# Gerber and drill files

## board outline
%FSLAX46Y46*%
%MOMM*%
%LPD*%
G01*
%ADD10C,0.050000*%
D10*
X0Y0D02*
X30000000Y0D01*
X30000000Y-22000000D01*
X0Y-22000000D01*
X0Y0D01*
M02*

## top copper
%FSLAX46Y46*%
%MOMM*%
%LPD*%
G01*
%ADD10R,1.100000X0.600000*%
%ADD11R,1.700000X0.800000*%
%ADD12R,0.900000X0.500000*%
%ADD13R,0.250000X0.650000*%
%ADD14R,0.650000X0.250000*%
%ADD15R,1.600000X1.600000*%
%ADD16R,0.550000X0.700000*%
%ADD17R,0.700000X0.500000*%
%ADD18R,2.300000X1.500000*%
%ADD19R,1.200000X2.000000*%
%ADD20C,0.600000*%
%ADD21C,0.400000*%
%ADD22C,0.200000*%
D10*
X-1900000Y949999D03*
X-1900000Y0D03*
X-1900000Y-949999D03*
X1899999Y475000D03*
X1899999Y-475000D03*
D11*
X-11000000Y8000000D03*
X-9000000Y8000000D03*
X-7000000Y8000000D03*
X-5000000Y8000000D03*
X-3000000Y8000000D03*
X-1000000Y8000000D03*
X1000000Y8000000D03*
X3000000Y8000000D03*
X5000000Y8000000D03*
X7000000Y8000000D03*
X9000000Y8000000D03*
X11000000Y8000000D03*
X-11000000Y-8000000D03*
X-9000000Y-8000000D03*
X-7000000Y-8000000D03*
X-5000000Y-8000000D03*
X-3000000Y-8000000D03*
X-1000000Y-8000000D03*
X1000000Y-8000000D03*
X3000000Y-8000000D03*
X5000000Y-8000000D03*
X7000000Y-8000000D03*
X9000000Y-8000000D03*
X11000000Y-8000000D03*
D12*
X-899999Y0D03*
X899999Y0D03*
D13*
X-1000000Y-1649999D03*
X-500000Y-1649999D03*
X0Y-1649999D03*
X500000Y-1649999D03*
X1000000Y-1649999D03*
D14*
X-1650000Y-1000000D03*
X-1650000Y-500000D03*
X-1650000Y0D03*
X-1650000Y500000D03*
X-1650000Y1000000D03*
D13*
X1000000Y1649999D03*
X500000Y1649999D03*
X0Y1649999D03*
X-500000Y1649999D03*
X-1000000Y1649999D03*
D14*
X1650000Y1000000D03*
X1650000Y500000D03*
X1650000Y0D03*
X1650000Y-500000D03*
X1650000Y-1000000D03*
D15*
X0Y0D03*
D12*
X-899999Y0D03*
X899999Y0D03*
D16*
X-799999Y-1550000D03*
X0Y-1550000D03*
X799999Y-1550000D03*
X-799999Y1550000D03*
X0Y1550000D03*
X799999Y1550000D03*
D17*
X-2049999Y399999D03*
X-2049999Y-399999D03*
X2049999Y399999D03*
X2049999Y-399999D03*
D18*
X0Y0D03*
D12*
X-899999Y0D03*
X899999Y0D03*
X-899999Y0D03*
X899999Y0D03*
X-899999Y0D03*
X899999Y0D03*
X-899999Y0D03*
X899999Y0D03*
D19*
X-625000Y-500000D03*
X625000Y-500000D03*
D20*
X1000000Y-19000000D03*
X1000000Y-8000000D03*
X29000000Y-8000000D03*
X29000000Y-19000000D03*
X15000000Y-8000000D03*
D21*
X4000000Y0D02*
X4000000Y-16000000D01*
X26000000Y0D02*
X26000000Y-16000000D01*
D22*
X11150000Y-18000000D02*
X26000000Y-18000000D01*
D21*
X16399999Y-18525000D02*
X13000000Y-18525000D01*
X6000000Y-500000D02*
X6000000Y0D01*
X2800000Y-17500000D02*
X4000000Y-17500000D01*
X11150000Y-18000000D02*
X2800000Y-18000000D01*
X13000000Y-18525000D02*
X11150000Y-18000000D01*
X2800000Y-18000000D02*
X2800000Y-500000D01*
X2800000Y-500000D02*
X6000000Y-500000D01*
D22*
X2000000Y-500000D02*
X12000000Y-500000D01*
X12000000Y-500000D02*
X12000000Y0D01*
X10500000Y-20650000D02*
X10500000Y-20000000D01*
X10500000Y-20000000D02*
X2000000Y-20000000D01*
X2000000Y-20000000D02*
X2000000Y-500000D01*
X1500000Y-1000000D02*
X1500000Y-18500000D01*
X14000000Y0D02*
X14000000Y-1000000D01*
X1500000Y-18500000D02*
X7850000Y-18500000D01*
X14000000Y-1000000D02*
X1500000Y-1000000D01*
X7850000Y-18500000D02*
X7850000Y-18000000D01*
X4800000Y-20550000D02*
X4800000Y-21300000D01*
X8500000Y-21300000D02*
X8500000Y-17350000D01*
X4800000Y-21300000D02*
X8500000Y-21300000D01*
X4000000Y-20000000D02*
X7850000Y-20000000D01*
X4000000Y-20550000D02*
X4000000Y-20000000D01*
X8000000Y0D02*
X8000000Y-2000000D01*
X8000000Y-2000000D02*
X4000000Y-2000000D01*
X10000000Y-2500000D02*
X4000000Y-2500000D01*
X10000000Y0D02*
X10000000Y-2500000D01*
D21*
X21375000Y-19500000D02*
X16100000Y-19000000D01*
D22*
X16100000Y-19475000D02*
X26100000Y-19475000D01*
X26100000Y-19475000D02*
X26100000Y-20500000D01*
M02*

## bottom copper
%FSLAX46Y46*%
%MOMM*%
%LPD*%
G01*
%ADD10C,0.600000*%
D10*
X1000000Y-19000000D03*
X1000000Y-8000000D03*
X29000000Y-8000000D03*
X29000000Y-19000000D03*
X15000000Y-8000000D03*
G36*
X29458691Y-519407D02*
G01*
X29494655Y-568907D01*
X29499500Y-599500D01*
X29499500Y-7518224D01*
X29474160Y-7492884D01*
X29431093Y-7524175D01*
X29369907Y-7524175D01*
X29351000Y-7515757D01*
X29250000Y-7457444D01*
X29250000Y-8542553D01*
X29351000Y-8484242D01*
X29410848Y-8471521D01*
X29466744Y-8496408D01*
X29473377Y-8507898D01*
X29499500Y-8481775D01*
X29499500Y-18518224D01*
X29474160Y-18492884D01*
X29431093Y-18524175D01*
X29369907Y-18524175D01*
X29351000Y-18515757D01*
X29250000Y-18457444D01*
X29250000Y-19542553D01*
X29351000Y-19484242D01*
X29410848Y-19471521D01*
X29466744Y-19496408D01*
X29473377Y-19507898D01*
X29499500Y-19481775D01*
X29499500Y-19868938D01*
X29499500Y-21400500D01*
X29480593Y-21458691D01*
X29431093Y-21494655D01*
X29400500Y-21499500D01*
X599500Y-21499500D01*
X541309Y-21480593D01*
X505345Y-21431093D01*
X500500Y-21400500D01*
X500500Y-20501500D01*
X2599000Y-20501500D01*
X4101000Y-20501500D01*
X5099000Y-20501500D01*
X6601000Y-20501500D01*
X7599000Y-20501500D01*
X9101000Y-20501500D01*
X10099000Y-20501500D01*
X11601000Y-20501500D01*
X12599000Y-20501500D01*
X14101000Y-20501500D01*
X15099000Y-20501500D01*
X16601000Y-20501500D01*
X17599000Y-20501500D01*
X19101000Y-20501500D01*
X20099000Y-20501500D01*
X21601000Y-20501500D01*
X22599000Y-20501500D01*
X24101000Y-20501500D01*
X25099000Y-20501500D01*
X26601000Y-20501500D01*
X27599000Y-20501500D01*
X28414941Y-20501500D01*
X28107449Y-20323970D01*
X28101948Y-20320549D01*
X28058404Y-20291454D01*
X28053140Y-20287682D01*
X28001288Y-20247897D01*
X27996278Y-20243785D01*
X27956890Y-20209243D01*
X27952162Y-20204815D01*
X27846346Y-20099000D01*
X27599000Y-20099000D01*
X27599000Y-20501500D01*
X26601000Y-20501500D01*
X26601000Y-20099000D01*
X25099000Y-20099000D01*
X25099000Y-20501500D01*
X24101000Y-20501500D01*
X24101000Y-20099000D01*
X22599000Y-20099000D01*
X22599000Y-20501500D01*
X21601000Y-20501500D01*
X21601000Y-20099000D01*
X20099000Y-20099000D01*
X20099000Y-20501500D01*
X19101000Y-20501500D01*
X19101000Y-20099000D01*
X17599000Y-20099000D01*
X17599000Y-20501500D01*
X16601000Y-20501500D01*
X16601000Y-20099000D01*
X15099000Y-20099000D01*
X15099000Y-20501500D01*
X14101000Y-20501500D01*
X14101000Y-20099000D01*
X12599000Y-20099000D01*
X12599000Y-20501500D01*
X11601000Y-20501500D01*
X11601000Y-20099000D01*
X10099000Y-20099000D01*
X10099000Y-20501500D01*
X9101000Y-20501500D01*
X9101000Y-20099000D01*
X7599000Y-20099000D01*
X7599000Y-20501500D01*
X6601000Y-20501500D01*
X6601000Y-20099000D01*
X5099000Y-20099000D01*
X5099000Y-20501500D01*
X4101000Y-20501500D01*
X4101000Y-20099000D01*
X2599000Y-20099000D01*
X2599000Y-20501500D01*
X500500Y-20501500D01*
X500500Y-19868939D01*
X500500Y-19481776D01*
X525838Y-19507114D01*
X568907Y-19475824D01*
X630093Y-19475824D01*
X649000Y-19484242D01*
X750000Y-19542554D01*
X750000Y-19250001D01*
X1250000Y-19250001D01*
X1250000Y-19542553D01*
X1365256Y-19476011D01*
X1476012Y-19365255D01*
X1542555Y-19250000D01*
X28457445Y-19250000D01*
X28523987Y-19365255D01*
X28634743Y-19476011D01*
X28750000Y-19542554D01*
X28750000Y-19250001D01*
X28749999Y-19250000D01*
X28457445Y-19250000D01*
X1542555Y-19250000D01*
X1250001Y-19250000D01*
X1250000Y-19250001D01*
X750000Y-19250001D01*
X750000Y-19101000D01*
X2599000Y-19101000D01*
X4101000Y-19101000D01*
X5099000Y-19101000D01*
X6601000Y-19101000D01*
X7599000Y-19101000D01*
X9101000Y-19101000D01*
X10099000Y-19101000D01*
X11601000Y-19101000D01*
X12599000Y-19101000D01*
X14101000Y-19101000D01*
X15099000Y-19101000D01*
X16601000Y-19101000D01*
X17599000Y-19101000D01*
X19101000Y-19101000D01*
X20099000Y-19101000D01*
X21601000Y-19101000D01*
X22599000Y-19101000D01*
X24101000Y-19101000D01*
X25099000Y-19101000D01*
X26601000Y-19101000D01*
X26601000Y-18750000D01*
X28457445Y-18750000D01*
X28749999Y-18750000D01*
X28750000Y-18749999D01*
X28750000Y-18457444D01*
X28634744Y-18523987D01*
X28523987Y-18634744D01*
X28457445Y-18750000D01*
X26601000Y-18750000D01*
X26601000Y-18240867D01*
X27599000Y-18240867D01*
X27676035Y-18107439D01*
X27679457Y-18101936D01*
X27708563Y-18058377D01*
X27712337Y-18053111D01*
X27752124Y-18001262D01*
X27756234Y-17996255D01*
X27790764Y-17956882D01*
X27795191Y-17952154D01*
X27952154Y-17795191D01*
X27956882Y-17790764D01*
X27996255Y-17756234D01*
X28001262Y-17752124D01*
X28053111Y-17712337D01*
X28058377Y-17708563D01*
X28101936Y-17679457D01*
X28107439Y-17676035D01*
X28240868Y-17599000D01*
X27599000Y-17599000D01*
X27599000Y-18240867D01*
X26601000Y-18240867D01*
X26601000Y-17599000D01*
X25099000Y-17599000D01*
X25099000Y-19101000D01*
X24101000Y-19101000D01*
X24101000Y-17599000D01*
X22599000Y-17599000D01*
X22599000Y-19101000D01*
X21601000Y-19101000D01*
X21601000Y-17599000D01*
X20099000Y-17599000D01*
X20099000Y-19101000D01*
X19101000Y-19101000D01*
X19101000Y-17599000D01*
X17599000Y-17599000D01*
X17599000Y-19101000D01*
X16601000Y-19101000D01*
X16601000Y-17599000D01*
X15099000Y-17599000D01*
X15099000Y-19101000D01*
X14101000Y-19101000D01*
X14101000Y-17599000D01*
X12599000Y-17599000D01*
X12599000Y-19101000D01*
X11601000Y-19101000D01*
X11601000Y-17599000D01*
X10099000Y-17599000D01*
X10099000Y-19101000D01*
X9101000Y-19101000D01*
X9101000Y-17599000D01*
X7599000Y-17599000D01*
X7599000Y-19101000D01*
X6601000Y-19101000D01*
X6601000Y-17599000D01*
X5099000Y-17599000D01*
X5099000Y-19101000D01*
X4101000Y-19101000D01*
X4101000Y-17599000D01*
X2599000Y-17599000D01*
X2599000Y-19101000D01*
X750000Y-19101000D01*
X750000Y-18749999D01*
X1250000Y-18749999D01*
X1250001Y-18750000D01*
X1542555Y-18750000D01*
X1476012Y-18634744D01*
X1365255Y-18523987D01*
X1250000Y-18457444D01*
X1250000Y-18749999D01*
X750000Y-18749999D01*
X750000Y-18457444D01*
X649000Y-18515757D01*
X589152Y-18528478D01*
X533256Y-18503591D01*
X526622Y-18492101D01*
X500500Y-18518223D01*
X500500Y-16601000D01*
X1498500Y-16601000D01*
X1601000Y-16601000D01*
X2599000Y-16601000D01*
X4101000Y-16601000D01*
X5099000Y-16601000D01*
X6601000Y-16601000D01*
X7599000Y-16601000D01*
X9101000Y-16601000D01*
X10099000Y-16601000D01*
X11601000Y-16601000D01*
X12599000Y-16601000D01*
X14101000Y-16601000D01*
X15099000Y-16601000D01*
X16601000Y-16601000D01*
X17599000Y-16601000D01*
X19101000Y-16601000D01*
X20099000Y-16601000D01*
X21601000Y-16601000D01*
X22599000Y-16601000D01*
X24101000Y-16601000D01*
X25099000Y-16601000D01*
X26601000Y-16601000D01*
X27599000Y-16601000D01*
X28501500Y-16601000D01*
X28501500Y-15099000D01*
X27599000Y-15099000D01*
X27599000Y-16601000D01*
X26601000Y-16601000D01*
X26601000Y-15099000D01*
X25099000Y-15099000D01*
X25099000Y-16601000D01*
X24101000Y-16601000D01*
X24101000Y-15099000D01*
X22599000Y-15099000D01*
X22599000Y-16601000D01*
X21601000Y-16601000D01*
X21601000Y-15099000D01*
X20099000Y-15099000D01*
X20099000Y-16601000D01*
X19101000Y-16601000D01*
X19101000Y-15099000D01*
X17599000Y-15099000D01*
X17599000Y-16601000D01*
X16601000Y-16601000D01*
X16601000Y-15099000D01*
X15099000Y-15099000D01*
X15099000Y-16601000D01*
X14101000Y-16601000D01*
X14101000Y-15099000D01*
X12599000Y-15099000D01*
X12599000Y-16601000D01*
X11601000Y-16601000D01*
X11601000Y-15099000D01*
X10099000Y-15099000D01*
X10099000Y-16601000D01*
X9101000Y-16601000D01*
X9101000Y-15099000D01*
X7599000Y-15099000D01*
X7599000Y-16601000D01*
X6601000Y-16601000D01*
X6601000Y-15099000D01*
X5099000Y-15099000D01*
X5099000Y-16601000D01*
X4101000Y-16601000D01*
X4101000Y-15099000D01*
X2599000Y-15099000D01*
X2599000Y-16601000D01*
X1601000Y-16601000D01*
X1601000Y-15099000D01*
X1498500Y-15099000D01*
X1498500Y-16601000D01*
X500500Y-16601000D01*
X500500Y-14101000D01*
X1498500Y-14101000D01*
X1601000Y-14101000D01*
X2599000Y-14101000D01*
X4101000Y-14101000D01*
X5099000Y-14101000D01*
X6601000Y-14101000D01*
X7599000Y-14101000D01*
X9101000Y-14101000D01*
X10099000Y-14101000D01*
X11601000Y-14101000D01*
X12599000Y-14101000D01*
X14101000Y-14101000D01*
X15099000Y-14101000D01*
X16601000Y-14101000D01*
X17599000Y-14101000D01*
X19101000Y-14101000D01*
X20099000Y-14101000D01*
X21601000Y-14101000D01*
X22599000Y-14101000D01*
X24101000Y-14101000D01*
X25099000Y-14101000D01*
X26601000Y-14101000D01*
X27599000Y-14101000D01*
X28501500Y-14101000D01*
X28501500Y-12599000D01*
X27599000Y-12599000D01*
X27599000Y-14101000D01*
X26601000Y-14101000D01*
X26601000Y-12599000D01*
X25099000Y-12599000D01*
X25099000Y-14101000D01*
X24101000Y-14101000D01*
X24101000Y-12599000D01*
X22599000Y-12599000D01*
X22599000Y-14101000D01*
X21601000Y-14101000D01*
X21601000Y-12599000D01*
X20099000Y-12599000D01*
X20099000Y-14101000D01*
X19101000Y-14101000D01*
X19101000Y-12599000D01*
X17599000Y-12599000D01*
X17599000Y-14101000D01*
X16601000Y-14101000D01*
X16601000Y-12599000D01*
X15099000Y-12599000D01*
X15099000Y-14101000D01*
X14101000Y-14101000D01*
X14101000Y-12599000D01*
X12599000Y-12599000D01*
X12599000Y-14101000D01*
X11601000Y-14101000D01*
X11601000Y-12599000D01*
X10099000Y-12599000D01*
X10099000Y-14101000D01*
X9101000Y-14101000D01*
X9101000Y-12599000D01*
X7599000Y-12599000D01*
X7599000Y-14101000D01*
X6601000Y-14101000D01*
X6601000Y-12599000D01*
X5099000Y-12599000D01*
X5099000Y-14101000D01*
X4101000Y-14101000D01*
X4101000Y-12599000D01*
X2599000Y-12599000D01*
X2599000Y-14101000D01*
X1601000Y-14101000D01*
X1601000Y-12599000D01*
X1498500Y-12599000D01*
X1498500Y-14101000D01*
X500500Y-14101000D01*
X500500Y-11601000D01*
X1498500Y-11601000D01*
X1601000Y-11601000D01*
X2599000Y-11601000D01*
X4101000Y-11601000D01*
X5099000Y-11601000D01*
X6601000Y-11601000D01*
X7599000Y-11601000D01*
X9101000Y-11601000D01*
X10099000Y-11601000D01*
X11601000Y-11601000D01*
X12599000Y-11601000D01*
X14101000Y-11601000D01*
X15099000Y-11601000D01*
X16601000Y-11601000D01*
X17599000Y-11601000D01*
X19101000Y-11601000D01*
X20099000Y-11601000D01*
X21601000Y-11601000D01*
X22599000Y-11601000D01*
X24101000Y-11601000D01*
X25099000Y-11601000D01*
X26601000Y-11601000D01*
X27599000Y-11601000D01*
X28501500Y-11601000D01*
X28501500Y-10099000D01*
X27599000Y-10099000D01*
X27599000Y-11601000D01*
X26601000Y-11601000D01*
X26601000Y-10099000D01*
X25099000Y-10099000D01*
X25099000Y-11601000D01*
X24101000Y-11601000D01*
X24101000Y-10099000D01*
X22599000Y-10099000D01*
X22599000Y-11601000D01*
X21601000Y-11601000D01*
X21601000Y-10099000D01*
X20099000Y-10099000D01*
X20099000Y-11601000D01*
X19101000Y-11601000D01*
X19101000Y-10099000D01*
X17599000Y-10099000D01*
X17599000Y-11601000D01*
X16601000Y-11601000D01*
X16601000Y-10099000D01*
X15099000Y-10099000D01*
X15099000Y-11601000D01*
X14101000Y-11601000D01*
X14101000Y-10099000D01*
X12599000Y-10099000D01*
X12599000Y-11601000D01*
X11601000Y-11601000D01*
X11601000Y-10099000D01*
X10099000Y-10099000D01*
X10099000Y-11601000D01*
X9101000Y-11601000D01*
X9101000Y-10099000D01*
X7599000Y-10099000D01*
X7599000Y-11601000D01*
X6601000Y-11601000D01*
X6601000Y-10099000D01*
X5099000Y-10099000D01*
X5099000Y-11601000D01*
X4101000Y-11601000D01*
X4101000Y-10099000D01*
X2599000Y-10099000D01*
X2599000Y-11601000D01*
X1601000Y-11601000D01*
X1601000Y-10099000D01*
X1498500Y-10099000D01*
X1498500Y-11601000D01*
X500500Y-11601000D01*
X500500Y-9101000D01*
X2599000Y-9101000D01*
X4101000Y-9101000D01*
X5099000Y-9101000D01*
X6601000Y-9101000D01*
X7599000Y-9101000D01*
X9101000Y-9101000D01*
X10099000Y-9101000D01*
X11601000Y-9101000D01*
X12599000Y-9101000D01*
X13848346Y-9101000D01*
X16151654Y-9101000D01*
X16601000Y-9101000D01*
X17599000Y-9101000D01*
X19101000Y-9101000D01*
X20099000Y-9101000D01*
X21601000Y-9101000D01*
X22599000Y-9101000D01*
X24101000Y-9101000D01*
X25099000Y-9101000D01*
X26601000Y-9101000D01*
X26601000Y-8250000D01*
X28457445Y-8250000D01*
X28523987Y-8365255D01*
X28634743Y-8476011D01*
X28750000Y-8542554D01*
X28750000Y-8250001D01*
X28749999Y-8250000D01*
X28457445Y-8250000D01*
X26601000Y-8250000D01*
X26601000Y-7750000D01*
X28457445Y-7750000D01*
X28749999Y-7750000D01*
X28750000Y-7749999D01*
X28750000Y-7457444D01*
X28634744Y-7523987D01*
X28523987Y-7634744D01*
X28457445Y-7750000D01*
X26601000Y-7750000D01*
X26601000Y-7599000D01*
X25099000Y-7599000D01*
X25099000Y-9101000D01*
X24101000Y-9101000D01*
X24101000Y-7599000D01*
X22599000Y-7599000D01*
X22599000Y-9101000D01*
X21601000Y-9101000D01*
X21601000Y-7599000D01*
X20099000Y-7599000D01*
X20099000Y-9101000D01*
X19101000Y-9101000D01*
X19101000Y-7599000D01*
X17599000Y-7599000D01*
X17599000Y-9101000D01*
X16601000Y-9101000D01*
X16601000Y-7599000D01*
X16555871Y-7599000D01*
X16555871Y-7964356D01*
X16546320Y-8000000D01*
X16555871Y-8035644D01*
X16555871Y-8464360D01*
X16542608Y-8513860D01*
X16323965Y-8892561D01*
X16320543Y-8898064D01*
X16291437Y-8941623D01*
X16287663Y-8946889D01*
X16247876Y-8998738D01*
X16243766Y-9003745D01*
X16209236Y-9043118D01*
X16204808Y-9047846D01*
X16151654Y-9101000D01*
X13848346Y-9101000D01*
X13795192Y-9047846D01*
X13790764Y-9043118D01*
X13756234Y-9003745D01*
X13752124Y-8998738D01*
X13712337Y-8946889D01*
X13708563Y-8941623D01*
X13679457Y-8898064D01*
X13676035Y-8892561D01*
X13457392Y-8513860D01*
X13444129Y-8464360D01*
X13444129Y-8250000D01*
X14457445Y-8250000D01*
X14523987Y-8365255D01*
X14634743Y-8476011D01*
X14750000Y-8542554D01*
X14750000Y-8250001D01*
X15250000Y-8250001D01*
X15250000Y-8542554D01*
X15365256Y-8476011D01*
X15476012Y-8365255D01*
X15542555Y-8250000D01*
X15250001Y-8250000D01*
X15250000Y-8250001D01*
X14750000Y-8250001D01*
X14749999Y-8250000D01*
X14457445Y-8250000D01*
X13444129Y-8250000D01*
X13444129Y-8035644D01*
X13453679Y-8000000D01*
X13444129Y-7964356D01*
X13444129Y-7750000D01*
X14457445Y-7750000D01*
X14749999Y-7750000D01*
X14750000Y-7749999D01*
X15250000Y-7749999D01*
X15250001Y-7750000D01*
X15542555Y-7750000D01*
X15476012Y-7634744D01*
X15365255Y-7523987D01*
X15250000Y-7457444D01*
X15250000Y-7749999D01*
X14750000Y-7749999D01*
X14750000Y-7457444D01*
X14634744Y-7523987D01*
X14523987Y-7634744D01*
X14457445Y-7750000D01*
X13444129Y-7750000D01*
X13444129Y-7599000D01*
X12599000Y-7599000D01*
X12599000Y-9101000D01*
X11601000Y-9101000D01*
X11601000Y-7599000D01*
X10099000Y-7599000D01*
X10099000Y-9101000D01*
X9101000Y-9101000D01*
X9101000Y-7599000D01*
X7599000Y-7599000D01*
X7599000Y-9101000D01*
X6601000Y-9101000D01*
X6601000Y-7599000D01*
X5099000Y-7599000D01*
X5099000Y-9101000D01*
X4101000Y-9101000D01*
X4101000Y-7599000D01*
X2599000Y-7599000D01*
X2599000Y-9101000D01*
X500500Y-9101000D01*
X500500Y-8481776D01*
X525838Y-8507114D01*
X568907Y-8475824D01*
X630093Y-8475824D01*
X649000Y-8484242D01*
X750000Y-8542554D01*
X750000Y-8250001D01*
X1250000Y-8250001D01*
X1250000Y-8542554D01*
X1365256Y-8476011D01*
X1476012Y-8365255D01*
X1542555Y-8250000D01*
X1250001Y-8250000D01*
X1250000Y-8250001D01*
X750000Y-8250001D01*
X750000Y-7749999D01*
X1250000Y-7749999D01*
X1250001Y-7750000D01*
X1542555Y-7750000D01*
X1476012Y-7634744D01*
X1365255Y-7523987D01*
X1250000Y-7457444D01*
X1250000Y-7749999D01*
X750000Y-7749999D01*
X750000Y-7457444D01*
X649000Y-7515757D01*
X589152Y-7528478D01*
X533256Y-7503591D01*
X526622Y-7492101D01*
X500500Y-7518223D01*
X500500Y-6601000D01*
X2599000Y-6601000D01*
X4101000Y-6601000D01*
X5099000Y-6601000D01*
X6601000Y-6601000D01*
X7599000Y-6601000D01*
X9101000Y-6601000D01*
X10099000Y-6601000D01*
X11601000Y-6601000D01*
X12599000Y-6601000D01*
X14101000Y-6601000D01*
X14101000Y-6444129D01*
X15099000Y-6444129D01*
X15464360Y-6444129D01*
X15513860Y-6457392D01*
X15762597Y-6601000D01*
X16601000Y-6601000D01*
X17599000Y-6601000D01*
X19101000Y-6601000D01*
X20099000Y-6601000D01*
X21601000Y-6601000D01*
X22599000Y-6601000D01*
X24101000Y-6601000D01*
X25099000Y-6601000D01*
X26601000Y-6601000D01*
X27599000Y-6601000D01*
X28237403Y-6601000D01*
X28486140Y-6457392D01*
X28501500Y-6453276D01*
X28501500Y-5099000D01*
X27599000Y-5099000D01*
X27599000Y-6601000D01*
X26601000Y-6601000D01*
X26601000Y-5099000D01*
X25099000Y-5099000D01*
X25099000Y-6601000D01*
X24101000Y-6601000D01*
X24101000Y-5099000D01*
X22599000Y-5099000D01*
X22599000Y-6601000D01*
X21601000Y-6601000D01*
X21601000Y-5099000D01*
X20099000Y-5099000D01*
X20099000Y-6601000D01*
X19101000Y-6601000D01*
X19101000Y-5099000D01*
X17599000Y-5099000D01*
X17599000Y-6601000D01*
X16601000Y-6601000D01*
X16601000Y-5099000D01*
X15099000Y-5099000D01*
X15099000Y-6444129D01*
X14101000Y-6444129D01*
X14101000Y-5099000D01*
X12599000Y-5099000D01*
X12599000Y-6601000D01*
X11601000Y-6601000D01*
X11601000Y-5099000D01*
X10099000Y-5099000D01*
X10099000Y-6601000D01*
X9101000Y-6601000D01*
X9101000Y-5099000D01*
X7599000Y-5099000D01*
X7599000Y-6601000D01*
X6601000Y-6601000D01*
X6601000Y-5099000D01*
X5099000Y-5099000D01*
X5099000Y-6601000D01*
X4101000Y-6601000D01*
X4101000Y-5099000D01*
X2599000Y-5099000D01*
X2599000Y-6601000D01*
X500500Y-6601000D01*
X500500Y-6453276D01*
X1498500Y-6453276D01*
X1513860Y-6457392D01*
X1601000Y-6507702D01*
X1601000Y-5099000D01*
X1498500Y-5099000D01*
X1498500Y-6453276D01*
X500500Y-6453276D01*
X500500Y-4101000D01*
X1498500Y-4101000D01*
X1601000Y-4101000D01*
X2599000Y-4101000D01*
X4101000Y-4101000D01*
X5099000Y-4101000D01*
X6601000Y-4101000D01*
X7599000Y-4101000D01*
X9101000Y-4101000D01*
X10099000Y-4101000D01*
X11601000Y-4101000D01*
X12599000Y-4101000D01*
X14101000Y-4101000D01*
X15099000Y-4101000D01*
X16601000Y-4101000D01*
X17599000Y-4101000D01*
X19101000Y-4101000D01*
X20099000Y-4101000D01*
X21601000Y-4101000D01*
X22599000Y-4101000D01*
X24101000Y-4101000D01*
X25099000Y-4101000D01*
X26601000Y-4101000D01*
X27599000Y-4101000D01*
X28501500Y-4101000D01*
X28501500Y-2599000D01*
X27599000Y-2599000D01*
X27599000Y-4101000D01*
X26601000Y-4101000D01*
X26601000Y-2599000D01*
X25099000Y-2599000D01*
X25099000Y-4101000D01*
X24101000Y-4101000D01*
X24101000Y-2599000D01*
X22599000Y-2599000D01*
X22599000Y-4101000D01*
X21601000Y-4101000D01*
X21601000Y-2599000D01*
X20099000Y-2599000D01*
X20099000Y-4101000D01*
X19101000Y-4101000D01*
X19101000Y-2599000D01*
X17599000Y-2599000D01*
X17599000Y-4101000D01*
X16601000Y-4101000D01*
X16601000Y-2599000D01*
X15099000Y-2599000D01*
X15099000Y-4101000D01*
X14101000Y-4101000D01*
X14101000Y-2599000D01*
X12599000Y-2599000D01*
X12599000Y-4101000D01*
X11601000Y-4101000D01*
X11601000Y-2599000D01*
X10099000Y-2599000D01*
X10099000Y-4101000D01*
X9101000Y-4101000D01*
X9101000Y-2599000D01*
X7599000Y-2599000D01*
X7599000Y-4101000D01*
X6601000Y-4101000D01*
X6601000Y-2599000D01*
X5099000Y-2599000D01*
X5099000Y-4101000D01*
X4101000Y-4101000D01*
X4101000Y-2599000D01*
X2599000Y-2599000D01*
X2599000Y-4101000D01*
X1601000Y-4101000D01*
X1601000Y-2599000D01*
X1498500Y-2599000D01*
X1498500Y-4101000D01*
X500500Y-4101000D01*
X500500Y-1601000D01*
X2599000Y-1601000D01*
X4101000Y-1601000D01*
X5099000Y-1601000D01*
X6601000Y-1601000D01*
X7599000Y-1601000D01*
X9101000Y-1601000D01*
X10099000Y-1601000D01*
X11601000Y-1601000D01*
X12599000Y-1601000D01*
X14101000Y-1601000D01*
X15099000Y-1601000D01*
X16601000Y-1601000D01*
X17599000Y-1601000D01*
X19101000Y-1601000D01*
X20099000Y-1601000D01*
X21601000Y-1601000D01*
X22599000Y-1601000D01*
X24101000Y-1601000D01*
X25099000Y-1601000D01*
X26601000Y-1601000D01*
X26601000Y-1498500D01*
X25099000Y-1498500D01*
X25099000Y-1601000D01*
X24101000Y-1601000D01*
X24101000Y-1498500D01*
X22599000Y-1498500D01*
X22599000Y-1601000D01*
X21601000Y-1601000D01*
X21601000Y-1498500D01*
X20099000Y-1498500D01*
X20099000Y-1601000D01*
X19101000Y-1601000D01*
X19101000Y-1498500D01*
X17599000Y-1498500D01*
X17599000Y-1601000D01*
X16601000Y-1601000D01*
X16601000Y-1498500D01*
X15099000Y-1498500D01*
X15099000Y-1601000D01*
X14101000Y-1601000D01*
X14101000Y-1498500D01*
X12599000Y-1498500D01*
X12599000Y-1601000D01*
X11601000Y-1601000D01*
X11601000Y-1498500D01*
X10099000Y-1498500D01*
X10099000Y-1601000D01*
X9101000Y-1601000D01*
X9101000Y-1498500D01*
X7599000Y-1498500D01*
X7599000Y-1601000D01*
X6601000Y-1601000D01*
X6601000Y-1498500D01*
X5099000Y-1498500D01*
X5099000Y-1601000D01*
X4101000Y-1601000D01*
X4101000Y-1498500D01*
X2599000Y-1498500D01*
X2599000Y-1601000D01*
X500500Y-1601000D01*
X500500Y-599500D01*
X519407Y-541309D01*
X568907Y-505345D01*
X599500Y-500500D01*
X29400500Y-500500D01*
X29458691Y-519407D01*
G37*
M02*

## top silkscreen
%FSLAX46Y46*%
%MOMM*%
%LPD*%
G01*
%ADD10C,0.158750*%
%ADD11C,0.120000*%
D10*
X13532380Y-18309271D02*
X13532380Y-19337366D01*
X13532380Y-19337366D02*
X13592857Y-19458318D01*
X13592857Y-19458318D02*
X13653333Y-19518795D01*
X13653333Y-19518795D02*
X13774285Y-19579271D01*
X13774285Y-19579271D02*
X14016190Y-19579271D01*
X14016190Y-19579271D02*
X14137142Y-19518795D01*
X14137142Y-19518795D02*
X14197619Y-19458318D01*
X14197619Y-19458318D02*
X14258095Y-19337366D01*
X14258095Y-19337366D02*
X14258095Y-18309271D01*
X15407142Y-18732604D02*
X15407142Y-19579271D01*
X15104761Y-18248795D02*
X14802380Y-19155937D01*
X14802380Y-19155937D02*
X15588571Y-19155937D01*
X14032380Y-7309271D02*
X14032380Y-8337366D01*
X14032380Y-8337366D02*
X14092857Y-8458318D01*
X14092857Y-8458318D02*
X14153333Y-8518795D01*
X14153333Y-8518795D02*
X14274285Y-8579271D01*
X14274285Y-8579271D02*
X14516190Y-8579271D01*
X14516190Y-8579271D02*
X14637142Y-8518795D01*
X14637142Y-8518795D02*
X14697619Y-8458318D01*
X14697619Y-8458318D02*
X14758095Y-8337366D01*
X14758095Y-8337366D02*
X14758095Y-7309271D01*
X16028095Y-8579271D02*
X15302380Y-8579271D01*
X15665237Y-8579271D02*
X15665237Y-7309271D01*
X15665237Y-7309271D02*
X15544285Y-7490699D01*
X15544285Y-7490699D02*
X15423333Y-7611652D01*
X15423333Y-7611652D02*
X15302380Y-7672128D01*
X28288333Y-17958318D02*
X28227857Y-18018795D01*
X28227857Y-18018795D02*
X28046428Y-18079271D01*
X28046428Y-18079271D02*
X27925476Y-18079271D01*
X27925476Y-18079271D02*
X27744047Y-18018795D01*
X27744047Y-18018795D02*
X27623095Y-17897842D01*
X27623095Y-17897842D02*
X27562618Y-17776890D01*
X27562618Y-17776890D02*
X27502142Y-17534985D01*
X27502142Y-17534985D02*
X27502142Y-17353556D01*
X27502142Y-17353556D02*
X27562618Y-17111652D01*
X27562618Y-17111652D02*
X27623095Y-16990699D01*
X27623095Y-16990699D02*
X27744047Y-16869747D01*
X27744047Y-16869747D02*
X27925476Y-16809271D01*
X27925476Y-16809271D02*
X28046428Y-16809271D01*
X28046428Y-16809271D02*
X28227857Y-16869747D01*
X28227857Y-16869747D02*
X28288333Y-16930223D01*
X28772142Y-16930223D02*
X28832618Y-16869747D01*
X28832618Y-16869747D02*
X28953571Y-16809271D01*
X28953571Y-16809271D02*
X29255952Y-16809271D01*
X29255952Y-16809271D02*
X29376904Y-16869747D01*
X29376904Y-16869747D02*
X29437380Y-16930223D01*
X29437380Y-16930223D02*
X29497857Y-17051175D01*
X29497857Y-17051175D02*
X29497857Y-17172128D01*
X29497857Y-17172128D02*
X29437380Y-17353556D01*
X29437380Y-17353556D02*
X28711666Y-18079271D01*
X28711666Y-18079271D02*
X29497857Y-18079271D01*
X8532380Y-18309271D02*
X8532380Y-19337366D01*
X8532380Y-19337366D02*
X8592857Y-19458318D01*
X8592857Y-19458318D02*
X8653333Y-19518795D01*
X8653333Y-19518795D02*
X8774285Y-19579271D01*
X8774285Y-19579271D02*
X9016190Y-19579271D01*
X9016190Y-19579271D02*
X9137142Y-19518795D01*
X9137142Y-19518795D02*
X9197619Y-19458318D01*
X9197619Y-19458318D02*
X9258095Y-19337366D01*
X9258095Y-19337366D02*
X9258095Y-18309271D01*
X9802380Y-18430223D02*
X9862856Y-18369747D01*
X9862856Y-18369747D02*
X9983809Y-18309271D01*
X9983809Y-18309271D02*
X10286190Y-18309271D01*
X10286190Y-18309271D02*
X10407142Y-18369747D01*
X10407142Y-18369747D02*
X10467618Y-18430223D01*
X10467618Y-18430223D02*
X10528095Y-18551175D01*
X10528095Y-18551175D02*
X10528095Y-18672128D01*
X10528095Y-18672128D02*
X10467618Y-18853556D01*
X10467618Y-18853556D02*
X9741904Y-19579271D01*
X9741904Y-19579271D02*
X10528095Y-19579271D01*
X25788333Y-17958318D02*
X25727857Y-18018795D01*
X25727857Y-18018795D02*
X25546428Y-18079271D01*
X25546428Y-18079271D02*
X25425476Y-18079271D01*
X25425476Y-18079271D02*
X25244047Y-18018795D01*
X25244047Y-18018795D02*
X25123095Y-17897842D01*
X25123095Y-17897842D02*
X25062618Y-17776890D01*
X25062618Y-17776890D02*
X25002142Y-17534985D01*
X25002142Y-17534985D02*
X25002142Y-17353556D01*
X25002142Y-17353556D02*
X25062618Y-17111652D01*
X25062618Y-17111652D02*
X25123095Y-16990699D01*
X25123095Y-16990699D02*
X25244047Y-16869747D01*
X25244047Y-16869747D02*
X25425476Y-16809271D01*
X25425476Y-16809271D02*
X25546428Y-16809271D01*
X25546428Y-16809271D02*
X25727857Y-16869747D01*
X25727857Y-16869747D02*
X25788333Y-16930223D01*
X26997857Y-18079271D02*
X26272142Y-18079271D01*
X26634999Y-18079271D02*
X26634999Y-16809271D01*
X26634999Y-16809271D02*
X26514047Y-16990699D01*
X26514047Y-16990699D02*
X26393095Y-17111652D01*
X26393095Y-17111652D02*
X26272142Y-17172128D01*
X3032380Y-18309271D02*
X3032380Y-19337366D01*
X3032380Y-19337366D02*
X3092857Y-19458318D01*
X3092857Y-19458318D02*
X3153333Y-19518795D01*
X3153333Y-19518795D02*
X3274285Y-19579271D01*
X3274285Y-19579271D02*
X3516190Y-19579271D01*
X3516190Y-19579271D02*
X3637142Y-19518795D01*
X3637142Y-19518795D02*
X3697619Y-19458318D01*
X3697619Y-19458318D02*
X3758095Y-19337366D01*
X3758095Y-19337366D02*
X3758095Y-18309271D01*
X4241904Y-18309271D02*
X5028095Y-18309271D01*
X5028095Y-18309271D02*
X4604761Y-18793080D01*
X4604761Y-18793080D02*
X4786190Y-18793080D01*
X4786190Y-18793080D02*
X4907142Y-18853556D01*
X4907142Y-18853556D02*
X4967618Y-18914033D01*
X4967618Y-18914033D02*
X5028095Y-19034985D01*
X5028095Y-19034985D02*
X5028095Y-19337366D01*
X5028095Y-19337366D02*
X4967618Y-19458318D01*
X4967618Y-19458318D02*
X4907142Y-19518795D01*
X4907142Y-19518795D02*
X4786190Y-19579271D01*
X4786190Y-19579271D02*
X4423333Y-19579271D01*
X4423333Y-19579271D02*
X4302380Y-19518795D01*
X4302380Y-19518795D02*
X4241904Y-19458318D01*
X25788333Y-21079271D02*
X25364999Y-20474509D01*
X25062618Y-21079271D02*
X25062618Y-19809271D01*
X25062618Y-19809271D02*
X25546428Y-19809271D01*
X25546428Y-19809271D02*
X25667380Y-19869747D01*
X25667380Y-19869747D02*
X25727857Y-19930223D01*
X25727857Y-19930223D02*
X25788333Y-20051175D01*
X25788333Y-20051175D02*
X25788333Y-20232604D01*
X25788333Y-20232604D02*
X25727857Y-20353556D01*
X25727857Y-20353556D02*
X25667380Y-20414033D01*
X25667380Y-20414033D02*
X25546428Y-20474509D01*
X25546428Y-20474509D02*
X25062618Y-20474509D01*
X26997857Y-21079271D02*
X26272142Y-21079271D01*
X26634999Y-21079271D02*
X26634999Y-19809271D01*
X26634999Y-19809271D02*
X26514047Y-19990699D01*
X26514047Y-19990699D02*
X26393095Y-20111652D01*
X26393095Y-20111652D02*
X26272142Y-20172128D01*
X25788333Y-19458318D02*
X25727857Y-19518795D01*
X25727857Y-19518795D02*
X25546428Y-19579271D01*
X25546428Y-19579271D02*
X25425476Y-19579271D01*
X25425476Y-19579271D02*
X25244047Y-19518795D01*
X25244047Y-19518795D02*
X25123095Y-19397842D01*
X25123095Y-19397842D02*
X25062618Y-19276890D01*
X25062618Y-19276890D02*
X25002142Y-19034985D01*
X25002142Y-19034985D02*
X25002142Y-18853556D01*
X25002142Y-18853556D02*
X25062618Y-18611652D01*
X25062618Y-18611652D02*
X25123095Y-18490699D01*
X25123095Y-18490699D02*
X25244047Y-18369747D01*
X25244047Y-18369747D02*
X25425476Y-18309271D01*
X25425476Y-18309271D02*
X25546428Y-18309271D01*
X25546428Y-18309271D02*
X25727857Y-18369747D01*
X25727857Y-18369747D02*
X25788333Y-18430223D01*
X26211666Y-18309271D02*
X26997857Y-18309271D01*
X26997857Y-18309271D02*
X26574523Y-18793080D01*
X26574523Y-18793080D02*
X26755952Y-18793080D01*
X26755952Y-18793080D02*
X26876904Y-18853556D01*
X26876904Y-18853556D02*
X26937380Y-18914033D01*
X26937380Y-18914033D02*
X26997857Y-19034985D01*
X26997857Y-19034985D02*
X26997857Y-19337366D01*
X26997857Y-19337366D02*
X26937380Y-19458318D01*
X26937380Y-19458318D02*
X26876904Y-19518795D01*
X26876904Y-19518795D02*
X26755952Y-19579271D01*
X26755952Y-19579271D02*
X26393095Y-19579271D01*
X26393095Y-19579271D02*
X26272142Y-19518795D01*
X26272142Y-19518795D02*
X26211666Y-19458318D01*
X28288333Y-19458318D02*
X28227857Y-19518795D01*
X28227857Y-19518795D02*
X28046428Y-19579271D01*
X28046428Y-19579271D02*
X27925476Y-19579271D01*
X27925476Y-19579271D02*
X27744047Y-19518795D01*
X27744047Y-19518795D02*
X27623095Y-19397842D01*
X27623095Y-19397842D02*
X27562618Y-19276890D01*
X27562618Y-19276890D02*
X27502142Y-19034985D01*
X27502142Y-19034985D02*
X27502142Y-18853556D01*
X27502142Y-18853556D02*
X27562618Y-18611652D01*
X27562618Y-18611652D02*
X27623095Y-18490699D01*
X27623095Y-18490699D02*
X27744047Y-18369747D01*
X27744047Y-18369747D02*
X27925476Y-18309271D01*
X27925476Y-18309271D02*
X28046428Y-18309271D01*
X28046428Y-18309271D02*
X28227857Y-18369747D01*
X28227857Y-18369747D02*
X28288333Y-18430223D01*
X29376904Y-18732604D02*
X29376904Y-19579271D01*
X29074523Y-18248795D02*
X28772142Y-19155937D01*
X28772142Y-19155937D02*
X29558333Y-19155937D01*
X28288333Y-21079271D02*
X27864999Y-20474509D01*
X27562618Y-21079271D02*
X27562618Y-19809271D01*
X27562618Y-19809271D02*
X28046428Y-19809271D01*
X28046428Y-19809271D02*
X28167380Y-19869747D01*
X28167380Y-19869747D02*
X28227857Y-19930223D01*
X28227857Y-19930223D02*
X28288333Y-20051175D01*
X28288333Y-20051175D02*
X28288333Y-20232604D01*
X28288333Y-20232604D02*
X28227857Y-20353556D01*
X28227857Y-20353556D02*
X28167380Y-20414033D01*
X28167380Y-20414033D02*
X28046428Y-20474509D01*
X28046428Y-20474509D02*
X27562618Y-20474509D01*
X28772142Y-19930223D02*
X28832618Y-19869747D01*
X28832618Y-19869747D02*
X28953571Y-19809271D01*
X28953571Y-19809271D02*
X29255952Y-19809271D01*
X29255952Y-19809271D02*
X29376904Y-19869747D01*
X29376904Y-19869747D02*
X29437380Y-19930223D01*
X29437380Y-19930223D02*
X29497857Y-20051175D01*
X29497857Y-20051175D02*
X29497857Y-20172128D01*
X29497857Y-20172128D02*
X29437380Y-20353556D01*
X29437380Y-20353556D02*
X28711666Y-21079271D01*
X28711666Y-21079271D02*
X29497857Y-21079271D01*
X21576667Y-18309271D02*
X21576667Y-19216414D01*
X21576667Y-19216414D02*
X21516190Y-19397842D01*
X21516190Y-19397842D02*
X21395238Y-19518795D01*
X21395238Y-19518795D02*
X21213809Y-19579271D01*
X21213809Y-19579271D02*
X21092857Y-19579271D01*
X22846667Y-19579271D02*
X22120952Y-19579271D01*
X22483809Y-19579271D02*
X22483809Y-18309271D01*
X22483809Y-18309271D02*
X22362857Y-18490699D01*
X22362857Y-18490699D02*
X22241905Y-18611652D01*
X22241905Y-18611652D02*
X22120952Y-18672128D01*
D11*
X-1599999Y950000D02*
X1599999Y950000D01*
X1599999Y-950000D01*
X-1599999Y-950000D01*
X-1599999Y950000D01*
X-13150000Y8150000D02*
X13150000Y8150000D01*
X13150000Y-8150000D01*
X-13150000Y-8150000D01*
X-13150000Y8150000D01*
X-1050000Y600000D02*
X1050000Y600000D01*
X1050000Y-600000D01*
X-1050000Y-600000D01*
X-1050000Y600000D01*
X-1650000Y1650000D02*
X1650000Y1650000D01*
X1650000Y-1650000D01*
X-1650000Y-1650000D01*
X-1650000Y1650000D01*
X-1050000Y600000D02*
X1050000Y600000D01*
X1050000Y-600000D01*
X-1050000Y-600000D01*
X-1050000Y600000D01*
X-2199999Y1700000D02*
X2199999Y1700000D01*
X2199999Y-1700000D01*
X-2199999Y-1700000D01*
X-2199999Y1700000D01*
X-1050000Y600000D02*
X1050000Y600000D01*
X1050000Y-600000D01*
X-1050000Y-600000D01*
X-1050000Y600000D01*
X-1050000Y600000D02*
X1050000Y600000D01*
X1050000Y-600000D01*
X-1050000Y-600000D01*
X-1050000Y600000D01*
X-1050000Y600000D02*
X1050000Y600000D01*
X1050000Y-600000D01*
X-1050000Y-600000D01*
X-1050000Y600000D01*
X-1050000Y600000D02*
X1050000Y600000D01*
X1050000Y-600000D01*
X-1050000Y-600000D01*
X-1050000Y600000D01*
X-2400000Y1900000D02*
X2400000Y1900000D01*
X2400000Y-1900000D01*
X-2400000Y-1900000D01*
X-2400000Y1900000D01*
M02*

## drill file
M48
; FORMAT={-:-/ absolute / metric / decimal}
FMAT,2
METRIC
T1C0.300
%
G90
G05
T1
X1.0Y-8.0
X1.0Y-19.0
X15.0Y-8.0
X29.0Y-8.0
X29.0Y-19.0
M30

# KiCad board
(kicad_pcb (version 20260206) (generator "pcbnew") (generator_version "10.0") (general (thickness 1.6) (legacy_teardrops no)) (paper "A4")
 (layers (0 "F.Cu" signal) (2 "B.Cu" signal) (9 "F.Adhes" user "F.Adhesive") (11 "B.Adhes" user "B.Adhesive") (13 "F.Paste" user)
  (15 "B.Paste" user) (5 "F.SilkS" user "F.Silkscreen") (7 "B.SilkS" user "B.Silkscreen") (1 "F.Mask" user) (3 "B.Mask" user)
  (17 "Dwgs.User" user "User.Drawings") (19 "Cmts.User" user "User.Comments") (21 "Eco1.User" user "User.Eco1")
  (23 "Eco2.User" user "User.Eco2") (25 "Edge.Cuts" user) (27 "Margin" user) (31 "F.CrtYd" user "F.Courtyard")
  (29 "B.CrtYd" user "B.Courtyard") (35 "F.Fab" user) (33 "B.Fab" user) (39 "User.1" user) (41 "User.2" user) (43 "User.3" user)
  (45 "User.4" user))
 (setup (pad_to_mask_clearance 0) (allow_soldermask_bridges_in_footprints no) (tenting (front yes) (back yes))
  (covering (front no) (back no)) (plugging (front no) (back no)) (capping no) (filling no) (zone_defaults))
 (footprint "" (layer "F.Cu") (at 14.5 19)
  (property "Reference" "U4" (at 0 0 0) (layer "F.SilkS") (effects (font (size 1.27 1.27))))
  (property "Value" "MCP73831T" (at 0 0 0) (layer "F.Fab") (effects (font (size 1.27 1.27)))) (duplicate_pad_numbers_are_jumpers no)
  (fp_rect (start -16.099999 -19.95) (end -12.900001 -18.05) (stroke (width 0.12) (type default)) (fill no) (layer "F.SilkS"))
  (pad "1" smd rect (at -16.4 -19.949999) (size 1.1 0.6) (layers "F.Cu" "F.Mask" "F.Paste") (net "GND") (thermal_bridge_angle 45))
  (pad "2" smd rect (at -16.4 -19) (size 1.1 0.6) (layers "F.Cu" "F.Mask" "F.Paste") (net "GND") (thermal_bridge_angle 45))
  (pad "3" smd rect (at -16.4 -18.050001) (size 1.1 0.6) (layers "F.Cu" "F.Mask" "F.Paste") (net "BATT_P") (thermal_bridge_angle 45))
  (pad "4" smd rect (at -12.600001 -19.475) (size 1.1 0.6) (layers "F.Cu" "F.Mask" "F.Paste") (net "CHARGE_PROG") (thermal_bridge_angle 45))
  (pad "5" smd rect (at -12.600001 -18.525) (size 1.1 0.6) (layers "F.Cu" "F.Mask" "F.Paste") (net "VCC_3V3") (thermal_bridge_angle 45)))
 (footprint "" (layer "F.Cu") (at 15 8)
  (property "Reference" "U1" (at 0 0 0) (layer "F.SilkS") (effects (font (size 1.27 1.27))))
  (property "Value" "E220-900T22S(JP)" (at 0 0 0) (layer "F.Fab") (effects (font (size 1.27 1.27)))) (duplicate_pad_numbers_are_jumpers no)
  (fp_rect (start -28.15 -16.15) (end -1.85 0.15) (stroke (width 0.12) (type default)) (fill no) (layer "F.SilkS"))
  (pad "1" smd rect (at -26 -16) (size 1.7 0.8) (layers "F.Cu" "F.Mask" "F.Paste") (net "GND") (thermal_bridge_angle 45))
  (pad "2" smd rect (at -24 -16) (size 1.7 0.8) (layers "F.Cu" "F.Mask" "F.Paste") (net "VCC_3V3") (thermal_bridge_angle 45))
  (pad "3" smd rect (at -22 -16) (size 1.7 0.8) (layers "F.Cu" "F.Mask" "F.Paste") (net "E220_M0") (thermal_bridge_angle 45))
  (pad "4" smd rect (at -20 -16) (size 1.7 0.8) (layers "F.Cu" "F.Mask" "F.Paste") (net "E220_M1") (thermal_bridge_angle 45))
  (pad "5" smd rect (at -18 -16) (size 1.7 0.8) (layers "F.Cu" "F.Mask" "F.Paste") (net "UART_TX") (thermal_bridge_angle 45))
  (pad "6" smd rect (at -16 -16) (size 1.7 0.8) (layers "F.Cu" "F.Mask" "F.Paste") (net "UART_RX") (thermal_bridge_angle 45))
  (pad "7" smd rect (at -14 -16) (size 1.7 0.8) (layers "F.Cu" "F.Mask" "F.Paste") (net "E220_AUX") (thermal_bridge_angle 45))
  (pad "8" smd rect (at -12 -16) (size 1.7 0.8) (layers "F.Cu" "F.Mask" "F.Paste") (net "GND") (thermal_bridge_angle 45))
  (pad "9" smd rect (at -10 -16) (size 1.7 0.8) (layers "F.Cu" "F.Mask" "F.Paste") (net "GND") (thermal_bridge_angle 45))
  (pad "10" smd rect (at -8 -16) (size 1.7 0.8) (layers "F.Cu" "F.Mask" "F.Paste") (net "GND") (thermal_bridge_angle 45))
  (pad "11" smd rect (at -6 -16) (size 1.7 0.8) (layers "F.Cu" "F.Mask" "F.Paste") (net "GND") (thermal_bridge_angle 45))
  (pad "12" smd rect (at -4 -16) (size 1.7 0.8) (layers "F.Cu" "F.Mask" "F.Paste") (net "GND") (thermal_bridge_angle 45))
  (pad "13" smd rect (at -26 0) (size 1.7 0.8) (layers "F.Cu" "F.Mask" "F.Paste") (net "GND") (thermal_bridge_angle 45))
  (pad "14" smd rect (at -24 0) (size 1.7 0.8) (layers "F.Cu" "F.Mask" "F.Paste") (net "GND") (thermal_bridge_angle 45))
  (pad "15" smd rect (at -22 0) (size 1.7 0.8) (layers "F.Cu" "F.Mask" "F.Paste") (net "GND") (thermal_bridge_angle 45))
  (pad "16" smd rect (at -20 0) (size 1.7 0.8) (layers "F.Cu" "F.Mask" "F.Paste") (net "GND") (thermal_bridge_angle 45))
  (pad "17" smd rect (at -18 0) (size 1.7 0.8) (layers "F.Cu" "F.Mask" "F.Paste") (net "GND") (thermal_bridge_angle 45))
  (pad "18" smd rect (at -16 0) (size 1.7 0.8) (layers "F.Cu" "F.Mask" "F.Paste") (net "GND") (thermal_bridge_angle 45))
  (pad "19" smd rect (at -14 0) (size 1.7 0.8) (layers "F.Cu" "F.Mask" "F.Paste") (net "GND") (thermal_bridge_angle 45))
  (pad "20" smd rect (at -12 0) (size 1.7 0.8) (layers "F.Cu" "F.Mask" "F.Paste") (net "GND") (thermal_bridge_angle 45))
  (pad "21" smd rect (at -10 0) (size 1.7 0.8) (layers "F.Cu" "F.Mask" "F.Paste") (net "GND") (thermal_bridge_angle 45))
  (pad "22" smd rect (at -8 0) (size 1.7 0.8) (layers "F.Cu" "F.Mask" "F.Paste") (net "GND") (thermal_bridge_angle 45))
  (pad "23" smd rect (at -6 0) (size 1.7 0.8) (layers "F.Cu" "F.Mask" "F.Paste") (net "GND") (thermal_bridge_angle 45))
  (pad "24" smd rect (at -4 0) (size 1.7 0.8) (layers "F.Cu" "F.Mask" "F.Paste") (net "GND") (thermal_bridge_angle 45)))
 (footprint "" (layer "F.Cu") (at 28.5 17.5)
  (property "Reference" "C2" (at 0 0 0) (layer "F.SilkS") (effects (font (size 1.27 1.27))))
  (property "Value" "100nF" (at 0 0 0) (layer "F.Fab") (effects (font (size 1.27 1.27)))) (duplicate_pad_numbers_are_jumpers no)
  (fp_rect (start -29.55 -18.1) (end -27.45 -16.9) (stroke (width 0.12) (type default)) (fill no) (layer "F.SilkS"))
  (pad "1" smd rect (at -29.399999 -17.5) (size 0.9 0.5) (layers "F.Cu" "F.Mask" "F.Paste") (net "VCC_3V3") (thermal_bridge_angle 45))
  (pad "2" smd rect (at -27.600001 -17.5) (size 0.9 0.5) (layers "F.Cu" "F.Mask" "F.Paste") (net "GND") (thermal_bridge_angle 45)))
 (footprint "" (layer "F.Cu") (at 9.5 19)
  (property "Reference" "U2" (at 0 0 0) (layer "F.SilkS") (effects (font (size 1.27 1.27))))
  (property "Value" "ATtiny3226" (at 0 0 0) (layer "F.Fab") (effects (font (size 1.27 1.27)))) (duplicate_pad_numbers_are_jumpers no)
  (fp_rect (start -11.15 -20.65) (end -7.85 -17.35) (stroke (width 0.12) (type default)) (fill no) (layer "F.SilkS"))
  (pad "1" smd rect (at -10.5 -17.350001) (size 0.25 0.65) (layers "F.Cu" "F.Mask" "F.Paste") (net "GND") (thermal_bridge_angle 45))
  (pad "2" smd rect (at -10 -17.350001) (size 0.25 0.65) (layers "F.Cu" "F.Mask" "F.Paste") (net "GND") (thermal_bridge_angle 45))
  (pad "3" smd rect (at -9.5 -17.350001) (size 0.25 0.65) (layers "F.Cu" "F.Mask" "F.Paste") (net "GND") (thermal_bridge_angle 45))
  (pad "4" smd rect (at -9 -17.350001) (size 0.25 0.65) (layers "F.Cu" "F.Mask" "F.Paste") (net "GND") (thermal_bridge_angle 45))
  (pad "5" smd rect (at -8.5 -17.350001) (size 0.25 0.65) (layers "F.Cu" "F.Mask" "F.Paste") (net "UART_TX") (thermal_bridge_angle 45))
  (pad "6" smd rect (at -11.15 -18) (size 0.65 0.25) (layers "F.Cu" "F.Mask" "F.Paste") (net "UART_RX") (thermal_bridge_angle 45))
  (pad "7" smd rect (at -11.15 -18.5) (size 0.65 0.25) (layers "F.Cu" "F.Mask" "F.Paste") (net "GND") (thermal_bridge_angle 45))
  (pad "8" smd rect (at -11.15 -19) (size 0.65 0.25) (layers "F.Cu" "F.Mask" "F.Paste") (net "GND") (thermal_bridge_angle 45))
  (pad "9" smd rect (at -11.15 -19.5) (size 0.65 0.25) (layers "F.Cu" "F.Mask" "F.Paste") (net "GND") (thermal_bridge_angle 45))
  (pad "10" smd rect (at -11.15 -20) (size 0.65 0.25) (layers "F.Cu" "F.Mask" "F.Paste") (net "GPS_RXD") (thermal_bridge_angle 45))
  (pad "11" smd rect (at -8.5 -20.649999) (size 0.25 0.65) (layers "F.Cu" "F.Mask" "F.Paste") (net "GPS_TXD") (thermal_bridge_angle 45))
  (pad "12" smd rect (at -9 -20.649999) (size 0.25 0.65) (layers "F.Cu" "F.Mask" "F.Paste") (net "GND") (thermal_bridge_angle 45))
  (pad "13" smd rect (at -9.5 -20.649999) (size 0.25 0.65) (layers "F.Cu" "F.Mask" "F.Paste") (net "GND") (thermal_bridge_angle 45))
  (pad "14" smd rect (at -10 -20.649999) (size 0.25 0.65) (layers "F.Cu" "F.Mask" "F.Paste") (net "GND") (thermal_bridge_angle 45))
  (pad "15" smd rect (at -10.5 -20.649999) (size 0.25 0.65) (layers "F.Cu" "F.Mask" "F.Paste") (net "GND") (thermal_bridge_angle 45))
  (pad "16" smd rect (at -7.85 -20) (size 0.65 0.25) (layers "F.Cu" "F.Mask" "F.Paste") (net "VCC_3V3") (thermal_bridge_angle 45))
  (pad "17" smd rect (at -7.85 -19.5) (size 0.65 0.25) (layers "F.Cu" "F.Mask" "F.Paste") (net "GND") (thermal_bridge_angle 45))
  (pad "18" smd rect (at -7.85 -19) (size 0.65 0.25) (layers "F.Cu" "F.Mask" "F.Paste") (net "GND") (thermal_bridge_angle 45))
  (pad "19" smd rect (at -7.85 -18.5) (size 0.65 0.25) (layers "F.Cu" "F.Mask" "F.Paste") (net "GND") (thermal_bridge_angle 45))
  (pad "20" smd rect (at -7.85 -18) (size 0.65 0.25) (layers "F.Cu" "F.Mask" "F.Paste") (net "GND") (thermal_bridge_angle 45))
  (pad "EP" smd rect (at -9.5 -19) (size 1.6 1.6) (layers "F.Cu" "F.Mask" "F.Paste") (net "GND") (thermal_bridge_angle 45)))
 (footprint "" (layer "F.Cu") (at 26 17.5)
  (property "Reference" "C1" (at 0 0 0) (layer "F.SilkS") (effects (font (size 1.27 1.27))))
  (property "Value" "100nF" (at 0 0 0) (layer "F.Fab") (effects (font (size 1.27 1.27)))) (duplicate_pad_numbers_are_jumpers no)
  (fp_rect (start -27.05 -18.1) (end -24.95 -16.9) (stroke (width 0.12) (type default)) (fill no) (layer "F.SilkS"))
  (pad "1" smd rect (at -26.899999 -17.5) (size 0.9 0.5) (layers "F.Cu" "F.Mask" "F.Paste") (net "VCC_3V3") (thermal_bridge_angle 45))
  (pad "2" smd rect (at -25.100001 -17.5) (size 0.9 0.5) (layers "F.Cu" "F.Mask" "F.Paste") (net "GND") (thermal_bridge_angle 45)))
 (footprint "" (layer "F.Cu") (at 4 19)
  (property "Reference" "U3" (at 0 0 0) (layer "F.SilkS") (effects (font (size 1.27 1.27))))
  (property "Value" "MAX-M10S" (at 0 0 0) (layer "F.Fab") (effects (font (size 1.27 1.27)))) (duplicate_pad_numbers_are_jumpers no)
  (fp_rect (start -6.199999 -20.7) (end -1.800001 -17.3) (stroke (width 0.12) (type default)) (fill no) (layer "F.SilkS"))
  (pad "1" smd rect (at -4.799999 -17.45) (size 0.55 0.7) (layers "F.Cu" "F.Mask" "F.Paste") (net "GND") (thermal_bridge_angle 45))
  (pad "2" smd rect (at -4 -17.45) (size 0.55 0.7) (layers "F.Cu" "F.Mask" "F.Paste") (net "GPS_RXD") (thermal_bridge_angle 45))
  (pad "3" smd rect (at -3.200001 -17.45) (size 0.55 0.7) (layers "F.Cu" "F.Mask" "F.Paste") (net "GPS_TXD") (thermal_bridge_angle 45))
  (pad "4" smd rect (at -4.799999 -20.55) (size 0.55 0.7) (layers "F.Cu" "F.Mask" "F.Paste") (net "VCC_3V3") (thermal_bridge_angle 45))
  (pad "5" smd rect (at -4 -20.55) (size 0.55 0.7) (layers "F.Cu" "F.Mask" "F.Paste") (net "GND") (thermal_bridge_angle 45))
  (pad "6" smd rect (at -3.200001 -20.55) (size 0.55 0.7) (layers "F.Cu" "F.Mask" "F.Paste") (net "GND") (thermal_bridge_angle 45))
  (pad "7" smd rect (at -6.049999 -19.399999) (size 0.7 0.5) (layers "F.Cu" "F.Mask" "F.Paste") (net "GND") (thermal_bridge_angle 45))
  (pad "8" smd rect (at -6.049999 -18.600001) (size 0.7 0.5) (layers "F.Cu" "F.Mask" "F.Paste") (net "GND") (thermal_bridge_angle 45))
  (pad "9" smd rect (at -1.950001 -19.399999) (size 0.7 0.5) (layers "F.Cu" "F.Mask" "F.Paste") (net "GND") (thermal_bridge_angle 45))
  (pad "10" smd rect (at -1.950001 -18.600001) (size 0.7 0.5) (layers "F.Cu" "F.Mask" "F.Paste") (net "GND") (thermal_bridge_angle 45))
  (pad "EP" smd rect (at -4 -19) (size 2.3 1.5) (layers "F.Cu" "F.Mask" "F.Paste") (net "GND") (thermal_bridge_angle 45)))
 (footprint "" (layer "F.Cu") (at 26 20.5)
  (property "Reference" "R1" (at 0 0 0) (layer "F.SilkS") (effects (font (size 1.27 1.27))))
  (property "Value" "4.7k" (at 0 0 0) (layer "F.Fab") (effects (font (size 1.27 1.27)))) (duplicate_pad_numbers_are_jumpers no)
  (fp_rect (start -27.05 -21.1) (end -24.95 -19.9) (stroke (width 0.12) (type default)) (fill no) (layer "F.SilkS"))
  (pad "1" smd rect (at -26.899999 -20.5) (size 0.9 0.5) (layers "F.Cu" "F.Mask" "F.Paste") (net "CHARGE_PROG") (thermal_bridge_angle 45))
  (pad "2" smd rect (at -25.100001 -20.5) (size 0.9 0.5) (layers "F.Cu" "F.Mask" "F.Paste") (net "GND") (thermal_bridge_angle 45)))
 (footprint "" (layer "F.Cu") (at 26 19)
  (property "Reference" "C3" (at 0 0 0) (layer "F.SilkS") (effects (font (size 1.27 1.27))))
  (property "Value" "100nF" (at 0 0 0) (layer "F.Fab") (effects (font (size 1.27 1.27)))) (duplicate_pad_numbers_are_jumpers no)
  (fp_rect (start -27.05 -19.6) (end -24.95 -18.4) (stroke (width 0.12) (type default)) (fill no) (layer "F.SilkS"))
  (pad "1" smd rect (at -26.899999 -19) (size 0.9 0.5) (layers "F.Cu" "F.Mask" "F.Paste") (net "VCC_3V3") (thermal_bridge_angle 45))
  (pad "2" smd rect (at -25.100001 -19) (size 0.9 0.5) (layers "F.Cu" "F.Mask" "F.Paste") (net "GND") (thermal_bridge_angle 45)))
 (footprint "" (layer "F.Cu") (at 28.5 19)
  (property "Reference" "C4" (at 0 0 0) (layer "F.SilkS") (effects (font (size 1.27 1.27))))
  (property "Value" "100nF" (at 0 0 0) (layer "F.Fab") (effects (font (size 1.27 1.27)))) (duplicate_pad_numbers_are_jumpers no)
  (fp_rect (start -29.55 -19.6) (end -27.45 -18.4) (stroke (width 0.12) (type default)) (fill no) (layer "F.SilkS"))
  (pad "1" smd rect (at -29.399999 -19) (size 0.9 0.5) (layers "F.Cu" "F.Mask" "F.Paste") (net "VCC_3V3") (thermal_bridge_angle 45))
  (pad "2" smd rect (at -27.600001 -19) (size 0.9 0.5) (layers "F.Cu" "F.Mask" "F.Paste") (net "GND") (thermal_bridge_angle 45)))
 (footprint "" (layer "F.Cu") (at 28.5 20.5)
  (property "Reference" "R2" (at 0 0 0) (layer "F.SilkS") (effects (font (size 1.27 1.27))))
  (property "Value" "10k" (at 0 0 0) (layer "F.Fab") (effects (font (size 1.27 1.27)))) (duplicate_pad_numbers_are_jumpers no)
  (fp_rect (start -29.55 -21.1) (end -27.45 -19.9) (stroke (width 0.12) (type default)) (fill no) (layer "F.SilkS"))
  (pad "1" smd rect (at -29.399999 -20.5) (size 0.9 0.5) (layers "F.Cu" "F.Mask" "F.Paste") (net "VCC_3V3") (thermal_bridge_angle 45))
  (pad "2" smd rect (at -27.600001 -20.5) (size 0.9 0.5) (layers "F.Cu" "F.Mask" "F.Paste") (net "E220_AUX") (thermal_bridge_angle 45)))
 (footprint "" (layer "F.Cu") (at 22 19)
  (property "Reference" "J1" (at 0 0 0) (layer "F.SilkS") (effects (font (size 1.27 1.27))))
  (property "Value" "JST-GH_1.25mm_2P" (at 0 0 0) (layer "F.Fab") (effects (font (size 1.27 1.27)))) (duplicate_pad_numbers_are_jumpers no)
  (fp_rect (start -24.4 -20.9) (end -19.6 -17.1) (stroke (width 0.12) (type default)) (fill no) (layer "F.SilkS"))
  (pad "1" smd rect (at -22.625 -18.5) (size 1.2 2) (layers "F.Cu" "F.Mask" "F.Paste") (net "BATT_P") (thermal_bridge_angle 45))
  (pad "2" smd rect (at -21.375 -18.5) (size 1.2 2) (layers "F.Cu" "F.Mask" "F.Paste") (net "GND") (thermal_bridge_angle 45)))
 (gr_rect (start 0 0) (end 30 22) (stroke (width 0.05) (type default)) (fill no) (layer "Edge.Cuts"))
 (segment (start 4 0) (end 4 16) (width 0.4) (layer "F.Cu") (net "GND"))
 (segment (start 26 0) (end 26 16) (width 0.4) (layer "F.Cu") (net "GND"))
 (via (at 1 19) (size 0.6) (drill 0.3) (layers "F.Cu" "B.Cu") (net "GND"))
 (via (at 1 8) (size 0.6) (drill 0.3) (layers "F.Cu" "B.Cu") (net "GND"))
 (via (at 29 8) (size 0.6) (drill 0.3) (layers "F.Cu" "B.Cu") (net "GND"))
 (via (at 29 19) (size 0.6) (drill 0.3) (layers "F.Cu" "B.Cu") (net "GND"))
 (via (at 15 8) (size 0.6) (drill 0.3) (layers "F.Cu" "B.Cu") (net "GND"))
 (segment (start 11.15 18) (end 26 18) (width 0.2) (layer "F.Cu") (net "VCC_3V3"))
 (segment (start 16.399999 18.525) (end 13 18.525) (width 0.4) (layer "F.Cu") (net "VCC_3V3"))
 (segment (start 6 0.5) (end 6 0) (width 0.4) (layer "F.Cu") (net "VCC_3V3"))
 (segment (start 2.8 17.5) (end 4 17.5) (width 0.4) (layer "F.Cu") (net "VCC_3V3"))
 (segment (start 11.15 18) (end 2.8 18) (width 0.4) (layer "F.Cu") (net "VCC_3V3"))
 (segment (start 13 18.525) (end 11.15 18) (width 0.4) (layer "F.Cu") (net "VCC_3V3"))
 (segment (start 2.8 18) (end 2.8 0.5) (width 0.4) (layer "F.Cu") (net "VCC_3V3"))
 (segment (start 2.8 0.5) (end 6 0.5) (width 0.4) (layer "F.Cu") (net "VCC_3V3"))
 (segment (start 2 0.5) (end 12 0.5) (width 0.2) (layer "F.Cu") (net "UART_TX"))
 (segment (start 12 0.5) (end 12 0) (width 0.2) (layer "F.Cu") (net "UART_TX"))
 (segment (start 10.5 20.65) (end 10.5 20) (width 0.2) (layer "F.Cu") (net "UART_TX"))
 (segment (start 10.5 20) (end 2 20) (width 0.2) (layer "F.Cu") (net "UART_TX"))
 (segment (start 2 20) (end 2 0.5) (width 0.2) (layer "F.Cu") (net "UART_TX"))
 (segment (start 1.5 1) (end 1.5 18.5) (width 0.2) (layer "F.Cu") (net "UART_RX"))
 (segment (start 14 0) (end 14 1) (width 0.2) (layer "F.Cu") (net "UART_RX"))
 (segment (start 1.5 18.5) (end 7.85 18.5) (width 0.2) (layer "F.Cu") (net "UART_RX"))
 (segment (start 14 1) (end 1.5 1) (width 0.2) (layer "F.Cu") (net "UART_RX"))
 (segment (start 7.85 18.5) (end 7.85 18) (width 0.2) (layer "F.Cu") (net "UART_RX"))
 (segment (start 4.8 20.55) (end 4.8 21.3) (width 0.2) (layer "F.Cu") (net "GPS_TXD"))
 (segment (start 8.5 21.3) (end 8.5 17.35) (width 0.2) (layer "F.Cu") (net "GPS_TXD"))
 (segment (start 4.8 21.3) (end 8.5 21.3) (width 0.2) (layer "F.Cu") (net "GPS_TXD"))
 (segment (start 4 20) (end 7.85 20) (width 0.2) (layer "F.Cu") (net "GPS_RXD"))
 (segment (start 4 20.55) (end 4 20) (width 0.2) (layer "F.Cu") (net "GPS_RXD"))
 (segment (start 8 0) (end 8 2) (width 0.2) (layer "F.Cu") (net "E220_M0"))
 (segment (start 8 2) (end 4 2) (width 0.2) (layer "F.Cu") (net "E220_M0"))
 (segment (start 10 2.5) (end 4 2.5) (width 0.2) (layer "F.Cu") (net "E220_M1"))
 (segment (start 10 0) (end 10 2.5) (width 0.2) (layer "F.Cu") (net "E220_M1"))
 (segment (start 21.375 19.5) (end 16.1 19) (width 0.4) (layer "F.Cu") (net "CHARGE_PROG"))
 (segment (start 16.1 19.475) (end 26.1 19.475) (width 0.2) (layer "F.Cu") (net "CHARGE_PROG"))
 (segment (start 26.1 19.475) (end 26.1 20.5) (width 0.2) (layer "F.Cu") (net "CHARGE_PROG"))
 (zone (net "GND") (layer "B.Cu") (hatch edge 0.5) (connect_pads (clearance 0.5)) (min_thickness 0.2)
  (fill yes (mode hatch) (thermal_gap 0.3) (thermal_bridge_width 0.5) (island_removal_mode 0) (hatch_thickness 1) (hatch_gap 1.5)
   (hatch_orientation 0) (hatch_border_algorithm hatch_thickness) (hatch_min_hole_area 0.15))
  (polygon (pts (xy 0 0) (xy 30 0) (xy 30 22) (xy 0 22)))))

